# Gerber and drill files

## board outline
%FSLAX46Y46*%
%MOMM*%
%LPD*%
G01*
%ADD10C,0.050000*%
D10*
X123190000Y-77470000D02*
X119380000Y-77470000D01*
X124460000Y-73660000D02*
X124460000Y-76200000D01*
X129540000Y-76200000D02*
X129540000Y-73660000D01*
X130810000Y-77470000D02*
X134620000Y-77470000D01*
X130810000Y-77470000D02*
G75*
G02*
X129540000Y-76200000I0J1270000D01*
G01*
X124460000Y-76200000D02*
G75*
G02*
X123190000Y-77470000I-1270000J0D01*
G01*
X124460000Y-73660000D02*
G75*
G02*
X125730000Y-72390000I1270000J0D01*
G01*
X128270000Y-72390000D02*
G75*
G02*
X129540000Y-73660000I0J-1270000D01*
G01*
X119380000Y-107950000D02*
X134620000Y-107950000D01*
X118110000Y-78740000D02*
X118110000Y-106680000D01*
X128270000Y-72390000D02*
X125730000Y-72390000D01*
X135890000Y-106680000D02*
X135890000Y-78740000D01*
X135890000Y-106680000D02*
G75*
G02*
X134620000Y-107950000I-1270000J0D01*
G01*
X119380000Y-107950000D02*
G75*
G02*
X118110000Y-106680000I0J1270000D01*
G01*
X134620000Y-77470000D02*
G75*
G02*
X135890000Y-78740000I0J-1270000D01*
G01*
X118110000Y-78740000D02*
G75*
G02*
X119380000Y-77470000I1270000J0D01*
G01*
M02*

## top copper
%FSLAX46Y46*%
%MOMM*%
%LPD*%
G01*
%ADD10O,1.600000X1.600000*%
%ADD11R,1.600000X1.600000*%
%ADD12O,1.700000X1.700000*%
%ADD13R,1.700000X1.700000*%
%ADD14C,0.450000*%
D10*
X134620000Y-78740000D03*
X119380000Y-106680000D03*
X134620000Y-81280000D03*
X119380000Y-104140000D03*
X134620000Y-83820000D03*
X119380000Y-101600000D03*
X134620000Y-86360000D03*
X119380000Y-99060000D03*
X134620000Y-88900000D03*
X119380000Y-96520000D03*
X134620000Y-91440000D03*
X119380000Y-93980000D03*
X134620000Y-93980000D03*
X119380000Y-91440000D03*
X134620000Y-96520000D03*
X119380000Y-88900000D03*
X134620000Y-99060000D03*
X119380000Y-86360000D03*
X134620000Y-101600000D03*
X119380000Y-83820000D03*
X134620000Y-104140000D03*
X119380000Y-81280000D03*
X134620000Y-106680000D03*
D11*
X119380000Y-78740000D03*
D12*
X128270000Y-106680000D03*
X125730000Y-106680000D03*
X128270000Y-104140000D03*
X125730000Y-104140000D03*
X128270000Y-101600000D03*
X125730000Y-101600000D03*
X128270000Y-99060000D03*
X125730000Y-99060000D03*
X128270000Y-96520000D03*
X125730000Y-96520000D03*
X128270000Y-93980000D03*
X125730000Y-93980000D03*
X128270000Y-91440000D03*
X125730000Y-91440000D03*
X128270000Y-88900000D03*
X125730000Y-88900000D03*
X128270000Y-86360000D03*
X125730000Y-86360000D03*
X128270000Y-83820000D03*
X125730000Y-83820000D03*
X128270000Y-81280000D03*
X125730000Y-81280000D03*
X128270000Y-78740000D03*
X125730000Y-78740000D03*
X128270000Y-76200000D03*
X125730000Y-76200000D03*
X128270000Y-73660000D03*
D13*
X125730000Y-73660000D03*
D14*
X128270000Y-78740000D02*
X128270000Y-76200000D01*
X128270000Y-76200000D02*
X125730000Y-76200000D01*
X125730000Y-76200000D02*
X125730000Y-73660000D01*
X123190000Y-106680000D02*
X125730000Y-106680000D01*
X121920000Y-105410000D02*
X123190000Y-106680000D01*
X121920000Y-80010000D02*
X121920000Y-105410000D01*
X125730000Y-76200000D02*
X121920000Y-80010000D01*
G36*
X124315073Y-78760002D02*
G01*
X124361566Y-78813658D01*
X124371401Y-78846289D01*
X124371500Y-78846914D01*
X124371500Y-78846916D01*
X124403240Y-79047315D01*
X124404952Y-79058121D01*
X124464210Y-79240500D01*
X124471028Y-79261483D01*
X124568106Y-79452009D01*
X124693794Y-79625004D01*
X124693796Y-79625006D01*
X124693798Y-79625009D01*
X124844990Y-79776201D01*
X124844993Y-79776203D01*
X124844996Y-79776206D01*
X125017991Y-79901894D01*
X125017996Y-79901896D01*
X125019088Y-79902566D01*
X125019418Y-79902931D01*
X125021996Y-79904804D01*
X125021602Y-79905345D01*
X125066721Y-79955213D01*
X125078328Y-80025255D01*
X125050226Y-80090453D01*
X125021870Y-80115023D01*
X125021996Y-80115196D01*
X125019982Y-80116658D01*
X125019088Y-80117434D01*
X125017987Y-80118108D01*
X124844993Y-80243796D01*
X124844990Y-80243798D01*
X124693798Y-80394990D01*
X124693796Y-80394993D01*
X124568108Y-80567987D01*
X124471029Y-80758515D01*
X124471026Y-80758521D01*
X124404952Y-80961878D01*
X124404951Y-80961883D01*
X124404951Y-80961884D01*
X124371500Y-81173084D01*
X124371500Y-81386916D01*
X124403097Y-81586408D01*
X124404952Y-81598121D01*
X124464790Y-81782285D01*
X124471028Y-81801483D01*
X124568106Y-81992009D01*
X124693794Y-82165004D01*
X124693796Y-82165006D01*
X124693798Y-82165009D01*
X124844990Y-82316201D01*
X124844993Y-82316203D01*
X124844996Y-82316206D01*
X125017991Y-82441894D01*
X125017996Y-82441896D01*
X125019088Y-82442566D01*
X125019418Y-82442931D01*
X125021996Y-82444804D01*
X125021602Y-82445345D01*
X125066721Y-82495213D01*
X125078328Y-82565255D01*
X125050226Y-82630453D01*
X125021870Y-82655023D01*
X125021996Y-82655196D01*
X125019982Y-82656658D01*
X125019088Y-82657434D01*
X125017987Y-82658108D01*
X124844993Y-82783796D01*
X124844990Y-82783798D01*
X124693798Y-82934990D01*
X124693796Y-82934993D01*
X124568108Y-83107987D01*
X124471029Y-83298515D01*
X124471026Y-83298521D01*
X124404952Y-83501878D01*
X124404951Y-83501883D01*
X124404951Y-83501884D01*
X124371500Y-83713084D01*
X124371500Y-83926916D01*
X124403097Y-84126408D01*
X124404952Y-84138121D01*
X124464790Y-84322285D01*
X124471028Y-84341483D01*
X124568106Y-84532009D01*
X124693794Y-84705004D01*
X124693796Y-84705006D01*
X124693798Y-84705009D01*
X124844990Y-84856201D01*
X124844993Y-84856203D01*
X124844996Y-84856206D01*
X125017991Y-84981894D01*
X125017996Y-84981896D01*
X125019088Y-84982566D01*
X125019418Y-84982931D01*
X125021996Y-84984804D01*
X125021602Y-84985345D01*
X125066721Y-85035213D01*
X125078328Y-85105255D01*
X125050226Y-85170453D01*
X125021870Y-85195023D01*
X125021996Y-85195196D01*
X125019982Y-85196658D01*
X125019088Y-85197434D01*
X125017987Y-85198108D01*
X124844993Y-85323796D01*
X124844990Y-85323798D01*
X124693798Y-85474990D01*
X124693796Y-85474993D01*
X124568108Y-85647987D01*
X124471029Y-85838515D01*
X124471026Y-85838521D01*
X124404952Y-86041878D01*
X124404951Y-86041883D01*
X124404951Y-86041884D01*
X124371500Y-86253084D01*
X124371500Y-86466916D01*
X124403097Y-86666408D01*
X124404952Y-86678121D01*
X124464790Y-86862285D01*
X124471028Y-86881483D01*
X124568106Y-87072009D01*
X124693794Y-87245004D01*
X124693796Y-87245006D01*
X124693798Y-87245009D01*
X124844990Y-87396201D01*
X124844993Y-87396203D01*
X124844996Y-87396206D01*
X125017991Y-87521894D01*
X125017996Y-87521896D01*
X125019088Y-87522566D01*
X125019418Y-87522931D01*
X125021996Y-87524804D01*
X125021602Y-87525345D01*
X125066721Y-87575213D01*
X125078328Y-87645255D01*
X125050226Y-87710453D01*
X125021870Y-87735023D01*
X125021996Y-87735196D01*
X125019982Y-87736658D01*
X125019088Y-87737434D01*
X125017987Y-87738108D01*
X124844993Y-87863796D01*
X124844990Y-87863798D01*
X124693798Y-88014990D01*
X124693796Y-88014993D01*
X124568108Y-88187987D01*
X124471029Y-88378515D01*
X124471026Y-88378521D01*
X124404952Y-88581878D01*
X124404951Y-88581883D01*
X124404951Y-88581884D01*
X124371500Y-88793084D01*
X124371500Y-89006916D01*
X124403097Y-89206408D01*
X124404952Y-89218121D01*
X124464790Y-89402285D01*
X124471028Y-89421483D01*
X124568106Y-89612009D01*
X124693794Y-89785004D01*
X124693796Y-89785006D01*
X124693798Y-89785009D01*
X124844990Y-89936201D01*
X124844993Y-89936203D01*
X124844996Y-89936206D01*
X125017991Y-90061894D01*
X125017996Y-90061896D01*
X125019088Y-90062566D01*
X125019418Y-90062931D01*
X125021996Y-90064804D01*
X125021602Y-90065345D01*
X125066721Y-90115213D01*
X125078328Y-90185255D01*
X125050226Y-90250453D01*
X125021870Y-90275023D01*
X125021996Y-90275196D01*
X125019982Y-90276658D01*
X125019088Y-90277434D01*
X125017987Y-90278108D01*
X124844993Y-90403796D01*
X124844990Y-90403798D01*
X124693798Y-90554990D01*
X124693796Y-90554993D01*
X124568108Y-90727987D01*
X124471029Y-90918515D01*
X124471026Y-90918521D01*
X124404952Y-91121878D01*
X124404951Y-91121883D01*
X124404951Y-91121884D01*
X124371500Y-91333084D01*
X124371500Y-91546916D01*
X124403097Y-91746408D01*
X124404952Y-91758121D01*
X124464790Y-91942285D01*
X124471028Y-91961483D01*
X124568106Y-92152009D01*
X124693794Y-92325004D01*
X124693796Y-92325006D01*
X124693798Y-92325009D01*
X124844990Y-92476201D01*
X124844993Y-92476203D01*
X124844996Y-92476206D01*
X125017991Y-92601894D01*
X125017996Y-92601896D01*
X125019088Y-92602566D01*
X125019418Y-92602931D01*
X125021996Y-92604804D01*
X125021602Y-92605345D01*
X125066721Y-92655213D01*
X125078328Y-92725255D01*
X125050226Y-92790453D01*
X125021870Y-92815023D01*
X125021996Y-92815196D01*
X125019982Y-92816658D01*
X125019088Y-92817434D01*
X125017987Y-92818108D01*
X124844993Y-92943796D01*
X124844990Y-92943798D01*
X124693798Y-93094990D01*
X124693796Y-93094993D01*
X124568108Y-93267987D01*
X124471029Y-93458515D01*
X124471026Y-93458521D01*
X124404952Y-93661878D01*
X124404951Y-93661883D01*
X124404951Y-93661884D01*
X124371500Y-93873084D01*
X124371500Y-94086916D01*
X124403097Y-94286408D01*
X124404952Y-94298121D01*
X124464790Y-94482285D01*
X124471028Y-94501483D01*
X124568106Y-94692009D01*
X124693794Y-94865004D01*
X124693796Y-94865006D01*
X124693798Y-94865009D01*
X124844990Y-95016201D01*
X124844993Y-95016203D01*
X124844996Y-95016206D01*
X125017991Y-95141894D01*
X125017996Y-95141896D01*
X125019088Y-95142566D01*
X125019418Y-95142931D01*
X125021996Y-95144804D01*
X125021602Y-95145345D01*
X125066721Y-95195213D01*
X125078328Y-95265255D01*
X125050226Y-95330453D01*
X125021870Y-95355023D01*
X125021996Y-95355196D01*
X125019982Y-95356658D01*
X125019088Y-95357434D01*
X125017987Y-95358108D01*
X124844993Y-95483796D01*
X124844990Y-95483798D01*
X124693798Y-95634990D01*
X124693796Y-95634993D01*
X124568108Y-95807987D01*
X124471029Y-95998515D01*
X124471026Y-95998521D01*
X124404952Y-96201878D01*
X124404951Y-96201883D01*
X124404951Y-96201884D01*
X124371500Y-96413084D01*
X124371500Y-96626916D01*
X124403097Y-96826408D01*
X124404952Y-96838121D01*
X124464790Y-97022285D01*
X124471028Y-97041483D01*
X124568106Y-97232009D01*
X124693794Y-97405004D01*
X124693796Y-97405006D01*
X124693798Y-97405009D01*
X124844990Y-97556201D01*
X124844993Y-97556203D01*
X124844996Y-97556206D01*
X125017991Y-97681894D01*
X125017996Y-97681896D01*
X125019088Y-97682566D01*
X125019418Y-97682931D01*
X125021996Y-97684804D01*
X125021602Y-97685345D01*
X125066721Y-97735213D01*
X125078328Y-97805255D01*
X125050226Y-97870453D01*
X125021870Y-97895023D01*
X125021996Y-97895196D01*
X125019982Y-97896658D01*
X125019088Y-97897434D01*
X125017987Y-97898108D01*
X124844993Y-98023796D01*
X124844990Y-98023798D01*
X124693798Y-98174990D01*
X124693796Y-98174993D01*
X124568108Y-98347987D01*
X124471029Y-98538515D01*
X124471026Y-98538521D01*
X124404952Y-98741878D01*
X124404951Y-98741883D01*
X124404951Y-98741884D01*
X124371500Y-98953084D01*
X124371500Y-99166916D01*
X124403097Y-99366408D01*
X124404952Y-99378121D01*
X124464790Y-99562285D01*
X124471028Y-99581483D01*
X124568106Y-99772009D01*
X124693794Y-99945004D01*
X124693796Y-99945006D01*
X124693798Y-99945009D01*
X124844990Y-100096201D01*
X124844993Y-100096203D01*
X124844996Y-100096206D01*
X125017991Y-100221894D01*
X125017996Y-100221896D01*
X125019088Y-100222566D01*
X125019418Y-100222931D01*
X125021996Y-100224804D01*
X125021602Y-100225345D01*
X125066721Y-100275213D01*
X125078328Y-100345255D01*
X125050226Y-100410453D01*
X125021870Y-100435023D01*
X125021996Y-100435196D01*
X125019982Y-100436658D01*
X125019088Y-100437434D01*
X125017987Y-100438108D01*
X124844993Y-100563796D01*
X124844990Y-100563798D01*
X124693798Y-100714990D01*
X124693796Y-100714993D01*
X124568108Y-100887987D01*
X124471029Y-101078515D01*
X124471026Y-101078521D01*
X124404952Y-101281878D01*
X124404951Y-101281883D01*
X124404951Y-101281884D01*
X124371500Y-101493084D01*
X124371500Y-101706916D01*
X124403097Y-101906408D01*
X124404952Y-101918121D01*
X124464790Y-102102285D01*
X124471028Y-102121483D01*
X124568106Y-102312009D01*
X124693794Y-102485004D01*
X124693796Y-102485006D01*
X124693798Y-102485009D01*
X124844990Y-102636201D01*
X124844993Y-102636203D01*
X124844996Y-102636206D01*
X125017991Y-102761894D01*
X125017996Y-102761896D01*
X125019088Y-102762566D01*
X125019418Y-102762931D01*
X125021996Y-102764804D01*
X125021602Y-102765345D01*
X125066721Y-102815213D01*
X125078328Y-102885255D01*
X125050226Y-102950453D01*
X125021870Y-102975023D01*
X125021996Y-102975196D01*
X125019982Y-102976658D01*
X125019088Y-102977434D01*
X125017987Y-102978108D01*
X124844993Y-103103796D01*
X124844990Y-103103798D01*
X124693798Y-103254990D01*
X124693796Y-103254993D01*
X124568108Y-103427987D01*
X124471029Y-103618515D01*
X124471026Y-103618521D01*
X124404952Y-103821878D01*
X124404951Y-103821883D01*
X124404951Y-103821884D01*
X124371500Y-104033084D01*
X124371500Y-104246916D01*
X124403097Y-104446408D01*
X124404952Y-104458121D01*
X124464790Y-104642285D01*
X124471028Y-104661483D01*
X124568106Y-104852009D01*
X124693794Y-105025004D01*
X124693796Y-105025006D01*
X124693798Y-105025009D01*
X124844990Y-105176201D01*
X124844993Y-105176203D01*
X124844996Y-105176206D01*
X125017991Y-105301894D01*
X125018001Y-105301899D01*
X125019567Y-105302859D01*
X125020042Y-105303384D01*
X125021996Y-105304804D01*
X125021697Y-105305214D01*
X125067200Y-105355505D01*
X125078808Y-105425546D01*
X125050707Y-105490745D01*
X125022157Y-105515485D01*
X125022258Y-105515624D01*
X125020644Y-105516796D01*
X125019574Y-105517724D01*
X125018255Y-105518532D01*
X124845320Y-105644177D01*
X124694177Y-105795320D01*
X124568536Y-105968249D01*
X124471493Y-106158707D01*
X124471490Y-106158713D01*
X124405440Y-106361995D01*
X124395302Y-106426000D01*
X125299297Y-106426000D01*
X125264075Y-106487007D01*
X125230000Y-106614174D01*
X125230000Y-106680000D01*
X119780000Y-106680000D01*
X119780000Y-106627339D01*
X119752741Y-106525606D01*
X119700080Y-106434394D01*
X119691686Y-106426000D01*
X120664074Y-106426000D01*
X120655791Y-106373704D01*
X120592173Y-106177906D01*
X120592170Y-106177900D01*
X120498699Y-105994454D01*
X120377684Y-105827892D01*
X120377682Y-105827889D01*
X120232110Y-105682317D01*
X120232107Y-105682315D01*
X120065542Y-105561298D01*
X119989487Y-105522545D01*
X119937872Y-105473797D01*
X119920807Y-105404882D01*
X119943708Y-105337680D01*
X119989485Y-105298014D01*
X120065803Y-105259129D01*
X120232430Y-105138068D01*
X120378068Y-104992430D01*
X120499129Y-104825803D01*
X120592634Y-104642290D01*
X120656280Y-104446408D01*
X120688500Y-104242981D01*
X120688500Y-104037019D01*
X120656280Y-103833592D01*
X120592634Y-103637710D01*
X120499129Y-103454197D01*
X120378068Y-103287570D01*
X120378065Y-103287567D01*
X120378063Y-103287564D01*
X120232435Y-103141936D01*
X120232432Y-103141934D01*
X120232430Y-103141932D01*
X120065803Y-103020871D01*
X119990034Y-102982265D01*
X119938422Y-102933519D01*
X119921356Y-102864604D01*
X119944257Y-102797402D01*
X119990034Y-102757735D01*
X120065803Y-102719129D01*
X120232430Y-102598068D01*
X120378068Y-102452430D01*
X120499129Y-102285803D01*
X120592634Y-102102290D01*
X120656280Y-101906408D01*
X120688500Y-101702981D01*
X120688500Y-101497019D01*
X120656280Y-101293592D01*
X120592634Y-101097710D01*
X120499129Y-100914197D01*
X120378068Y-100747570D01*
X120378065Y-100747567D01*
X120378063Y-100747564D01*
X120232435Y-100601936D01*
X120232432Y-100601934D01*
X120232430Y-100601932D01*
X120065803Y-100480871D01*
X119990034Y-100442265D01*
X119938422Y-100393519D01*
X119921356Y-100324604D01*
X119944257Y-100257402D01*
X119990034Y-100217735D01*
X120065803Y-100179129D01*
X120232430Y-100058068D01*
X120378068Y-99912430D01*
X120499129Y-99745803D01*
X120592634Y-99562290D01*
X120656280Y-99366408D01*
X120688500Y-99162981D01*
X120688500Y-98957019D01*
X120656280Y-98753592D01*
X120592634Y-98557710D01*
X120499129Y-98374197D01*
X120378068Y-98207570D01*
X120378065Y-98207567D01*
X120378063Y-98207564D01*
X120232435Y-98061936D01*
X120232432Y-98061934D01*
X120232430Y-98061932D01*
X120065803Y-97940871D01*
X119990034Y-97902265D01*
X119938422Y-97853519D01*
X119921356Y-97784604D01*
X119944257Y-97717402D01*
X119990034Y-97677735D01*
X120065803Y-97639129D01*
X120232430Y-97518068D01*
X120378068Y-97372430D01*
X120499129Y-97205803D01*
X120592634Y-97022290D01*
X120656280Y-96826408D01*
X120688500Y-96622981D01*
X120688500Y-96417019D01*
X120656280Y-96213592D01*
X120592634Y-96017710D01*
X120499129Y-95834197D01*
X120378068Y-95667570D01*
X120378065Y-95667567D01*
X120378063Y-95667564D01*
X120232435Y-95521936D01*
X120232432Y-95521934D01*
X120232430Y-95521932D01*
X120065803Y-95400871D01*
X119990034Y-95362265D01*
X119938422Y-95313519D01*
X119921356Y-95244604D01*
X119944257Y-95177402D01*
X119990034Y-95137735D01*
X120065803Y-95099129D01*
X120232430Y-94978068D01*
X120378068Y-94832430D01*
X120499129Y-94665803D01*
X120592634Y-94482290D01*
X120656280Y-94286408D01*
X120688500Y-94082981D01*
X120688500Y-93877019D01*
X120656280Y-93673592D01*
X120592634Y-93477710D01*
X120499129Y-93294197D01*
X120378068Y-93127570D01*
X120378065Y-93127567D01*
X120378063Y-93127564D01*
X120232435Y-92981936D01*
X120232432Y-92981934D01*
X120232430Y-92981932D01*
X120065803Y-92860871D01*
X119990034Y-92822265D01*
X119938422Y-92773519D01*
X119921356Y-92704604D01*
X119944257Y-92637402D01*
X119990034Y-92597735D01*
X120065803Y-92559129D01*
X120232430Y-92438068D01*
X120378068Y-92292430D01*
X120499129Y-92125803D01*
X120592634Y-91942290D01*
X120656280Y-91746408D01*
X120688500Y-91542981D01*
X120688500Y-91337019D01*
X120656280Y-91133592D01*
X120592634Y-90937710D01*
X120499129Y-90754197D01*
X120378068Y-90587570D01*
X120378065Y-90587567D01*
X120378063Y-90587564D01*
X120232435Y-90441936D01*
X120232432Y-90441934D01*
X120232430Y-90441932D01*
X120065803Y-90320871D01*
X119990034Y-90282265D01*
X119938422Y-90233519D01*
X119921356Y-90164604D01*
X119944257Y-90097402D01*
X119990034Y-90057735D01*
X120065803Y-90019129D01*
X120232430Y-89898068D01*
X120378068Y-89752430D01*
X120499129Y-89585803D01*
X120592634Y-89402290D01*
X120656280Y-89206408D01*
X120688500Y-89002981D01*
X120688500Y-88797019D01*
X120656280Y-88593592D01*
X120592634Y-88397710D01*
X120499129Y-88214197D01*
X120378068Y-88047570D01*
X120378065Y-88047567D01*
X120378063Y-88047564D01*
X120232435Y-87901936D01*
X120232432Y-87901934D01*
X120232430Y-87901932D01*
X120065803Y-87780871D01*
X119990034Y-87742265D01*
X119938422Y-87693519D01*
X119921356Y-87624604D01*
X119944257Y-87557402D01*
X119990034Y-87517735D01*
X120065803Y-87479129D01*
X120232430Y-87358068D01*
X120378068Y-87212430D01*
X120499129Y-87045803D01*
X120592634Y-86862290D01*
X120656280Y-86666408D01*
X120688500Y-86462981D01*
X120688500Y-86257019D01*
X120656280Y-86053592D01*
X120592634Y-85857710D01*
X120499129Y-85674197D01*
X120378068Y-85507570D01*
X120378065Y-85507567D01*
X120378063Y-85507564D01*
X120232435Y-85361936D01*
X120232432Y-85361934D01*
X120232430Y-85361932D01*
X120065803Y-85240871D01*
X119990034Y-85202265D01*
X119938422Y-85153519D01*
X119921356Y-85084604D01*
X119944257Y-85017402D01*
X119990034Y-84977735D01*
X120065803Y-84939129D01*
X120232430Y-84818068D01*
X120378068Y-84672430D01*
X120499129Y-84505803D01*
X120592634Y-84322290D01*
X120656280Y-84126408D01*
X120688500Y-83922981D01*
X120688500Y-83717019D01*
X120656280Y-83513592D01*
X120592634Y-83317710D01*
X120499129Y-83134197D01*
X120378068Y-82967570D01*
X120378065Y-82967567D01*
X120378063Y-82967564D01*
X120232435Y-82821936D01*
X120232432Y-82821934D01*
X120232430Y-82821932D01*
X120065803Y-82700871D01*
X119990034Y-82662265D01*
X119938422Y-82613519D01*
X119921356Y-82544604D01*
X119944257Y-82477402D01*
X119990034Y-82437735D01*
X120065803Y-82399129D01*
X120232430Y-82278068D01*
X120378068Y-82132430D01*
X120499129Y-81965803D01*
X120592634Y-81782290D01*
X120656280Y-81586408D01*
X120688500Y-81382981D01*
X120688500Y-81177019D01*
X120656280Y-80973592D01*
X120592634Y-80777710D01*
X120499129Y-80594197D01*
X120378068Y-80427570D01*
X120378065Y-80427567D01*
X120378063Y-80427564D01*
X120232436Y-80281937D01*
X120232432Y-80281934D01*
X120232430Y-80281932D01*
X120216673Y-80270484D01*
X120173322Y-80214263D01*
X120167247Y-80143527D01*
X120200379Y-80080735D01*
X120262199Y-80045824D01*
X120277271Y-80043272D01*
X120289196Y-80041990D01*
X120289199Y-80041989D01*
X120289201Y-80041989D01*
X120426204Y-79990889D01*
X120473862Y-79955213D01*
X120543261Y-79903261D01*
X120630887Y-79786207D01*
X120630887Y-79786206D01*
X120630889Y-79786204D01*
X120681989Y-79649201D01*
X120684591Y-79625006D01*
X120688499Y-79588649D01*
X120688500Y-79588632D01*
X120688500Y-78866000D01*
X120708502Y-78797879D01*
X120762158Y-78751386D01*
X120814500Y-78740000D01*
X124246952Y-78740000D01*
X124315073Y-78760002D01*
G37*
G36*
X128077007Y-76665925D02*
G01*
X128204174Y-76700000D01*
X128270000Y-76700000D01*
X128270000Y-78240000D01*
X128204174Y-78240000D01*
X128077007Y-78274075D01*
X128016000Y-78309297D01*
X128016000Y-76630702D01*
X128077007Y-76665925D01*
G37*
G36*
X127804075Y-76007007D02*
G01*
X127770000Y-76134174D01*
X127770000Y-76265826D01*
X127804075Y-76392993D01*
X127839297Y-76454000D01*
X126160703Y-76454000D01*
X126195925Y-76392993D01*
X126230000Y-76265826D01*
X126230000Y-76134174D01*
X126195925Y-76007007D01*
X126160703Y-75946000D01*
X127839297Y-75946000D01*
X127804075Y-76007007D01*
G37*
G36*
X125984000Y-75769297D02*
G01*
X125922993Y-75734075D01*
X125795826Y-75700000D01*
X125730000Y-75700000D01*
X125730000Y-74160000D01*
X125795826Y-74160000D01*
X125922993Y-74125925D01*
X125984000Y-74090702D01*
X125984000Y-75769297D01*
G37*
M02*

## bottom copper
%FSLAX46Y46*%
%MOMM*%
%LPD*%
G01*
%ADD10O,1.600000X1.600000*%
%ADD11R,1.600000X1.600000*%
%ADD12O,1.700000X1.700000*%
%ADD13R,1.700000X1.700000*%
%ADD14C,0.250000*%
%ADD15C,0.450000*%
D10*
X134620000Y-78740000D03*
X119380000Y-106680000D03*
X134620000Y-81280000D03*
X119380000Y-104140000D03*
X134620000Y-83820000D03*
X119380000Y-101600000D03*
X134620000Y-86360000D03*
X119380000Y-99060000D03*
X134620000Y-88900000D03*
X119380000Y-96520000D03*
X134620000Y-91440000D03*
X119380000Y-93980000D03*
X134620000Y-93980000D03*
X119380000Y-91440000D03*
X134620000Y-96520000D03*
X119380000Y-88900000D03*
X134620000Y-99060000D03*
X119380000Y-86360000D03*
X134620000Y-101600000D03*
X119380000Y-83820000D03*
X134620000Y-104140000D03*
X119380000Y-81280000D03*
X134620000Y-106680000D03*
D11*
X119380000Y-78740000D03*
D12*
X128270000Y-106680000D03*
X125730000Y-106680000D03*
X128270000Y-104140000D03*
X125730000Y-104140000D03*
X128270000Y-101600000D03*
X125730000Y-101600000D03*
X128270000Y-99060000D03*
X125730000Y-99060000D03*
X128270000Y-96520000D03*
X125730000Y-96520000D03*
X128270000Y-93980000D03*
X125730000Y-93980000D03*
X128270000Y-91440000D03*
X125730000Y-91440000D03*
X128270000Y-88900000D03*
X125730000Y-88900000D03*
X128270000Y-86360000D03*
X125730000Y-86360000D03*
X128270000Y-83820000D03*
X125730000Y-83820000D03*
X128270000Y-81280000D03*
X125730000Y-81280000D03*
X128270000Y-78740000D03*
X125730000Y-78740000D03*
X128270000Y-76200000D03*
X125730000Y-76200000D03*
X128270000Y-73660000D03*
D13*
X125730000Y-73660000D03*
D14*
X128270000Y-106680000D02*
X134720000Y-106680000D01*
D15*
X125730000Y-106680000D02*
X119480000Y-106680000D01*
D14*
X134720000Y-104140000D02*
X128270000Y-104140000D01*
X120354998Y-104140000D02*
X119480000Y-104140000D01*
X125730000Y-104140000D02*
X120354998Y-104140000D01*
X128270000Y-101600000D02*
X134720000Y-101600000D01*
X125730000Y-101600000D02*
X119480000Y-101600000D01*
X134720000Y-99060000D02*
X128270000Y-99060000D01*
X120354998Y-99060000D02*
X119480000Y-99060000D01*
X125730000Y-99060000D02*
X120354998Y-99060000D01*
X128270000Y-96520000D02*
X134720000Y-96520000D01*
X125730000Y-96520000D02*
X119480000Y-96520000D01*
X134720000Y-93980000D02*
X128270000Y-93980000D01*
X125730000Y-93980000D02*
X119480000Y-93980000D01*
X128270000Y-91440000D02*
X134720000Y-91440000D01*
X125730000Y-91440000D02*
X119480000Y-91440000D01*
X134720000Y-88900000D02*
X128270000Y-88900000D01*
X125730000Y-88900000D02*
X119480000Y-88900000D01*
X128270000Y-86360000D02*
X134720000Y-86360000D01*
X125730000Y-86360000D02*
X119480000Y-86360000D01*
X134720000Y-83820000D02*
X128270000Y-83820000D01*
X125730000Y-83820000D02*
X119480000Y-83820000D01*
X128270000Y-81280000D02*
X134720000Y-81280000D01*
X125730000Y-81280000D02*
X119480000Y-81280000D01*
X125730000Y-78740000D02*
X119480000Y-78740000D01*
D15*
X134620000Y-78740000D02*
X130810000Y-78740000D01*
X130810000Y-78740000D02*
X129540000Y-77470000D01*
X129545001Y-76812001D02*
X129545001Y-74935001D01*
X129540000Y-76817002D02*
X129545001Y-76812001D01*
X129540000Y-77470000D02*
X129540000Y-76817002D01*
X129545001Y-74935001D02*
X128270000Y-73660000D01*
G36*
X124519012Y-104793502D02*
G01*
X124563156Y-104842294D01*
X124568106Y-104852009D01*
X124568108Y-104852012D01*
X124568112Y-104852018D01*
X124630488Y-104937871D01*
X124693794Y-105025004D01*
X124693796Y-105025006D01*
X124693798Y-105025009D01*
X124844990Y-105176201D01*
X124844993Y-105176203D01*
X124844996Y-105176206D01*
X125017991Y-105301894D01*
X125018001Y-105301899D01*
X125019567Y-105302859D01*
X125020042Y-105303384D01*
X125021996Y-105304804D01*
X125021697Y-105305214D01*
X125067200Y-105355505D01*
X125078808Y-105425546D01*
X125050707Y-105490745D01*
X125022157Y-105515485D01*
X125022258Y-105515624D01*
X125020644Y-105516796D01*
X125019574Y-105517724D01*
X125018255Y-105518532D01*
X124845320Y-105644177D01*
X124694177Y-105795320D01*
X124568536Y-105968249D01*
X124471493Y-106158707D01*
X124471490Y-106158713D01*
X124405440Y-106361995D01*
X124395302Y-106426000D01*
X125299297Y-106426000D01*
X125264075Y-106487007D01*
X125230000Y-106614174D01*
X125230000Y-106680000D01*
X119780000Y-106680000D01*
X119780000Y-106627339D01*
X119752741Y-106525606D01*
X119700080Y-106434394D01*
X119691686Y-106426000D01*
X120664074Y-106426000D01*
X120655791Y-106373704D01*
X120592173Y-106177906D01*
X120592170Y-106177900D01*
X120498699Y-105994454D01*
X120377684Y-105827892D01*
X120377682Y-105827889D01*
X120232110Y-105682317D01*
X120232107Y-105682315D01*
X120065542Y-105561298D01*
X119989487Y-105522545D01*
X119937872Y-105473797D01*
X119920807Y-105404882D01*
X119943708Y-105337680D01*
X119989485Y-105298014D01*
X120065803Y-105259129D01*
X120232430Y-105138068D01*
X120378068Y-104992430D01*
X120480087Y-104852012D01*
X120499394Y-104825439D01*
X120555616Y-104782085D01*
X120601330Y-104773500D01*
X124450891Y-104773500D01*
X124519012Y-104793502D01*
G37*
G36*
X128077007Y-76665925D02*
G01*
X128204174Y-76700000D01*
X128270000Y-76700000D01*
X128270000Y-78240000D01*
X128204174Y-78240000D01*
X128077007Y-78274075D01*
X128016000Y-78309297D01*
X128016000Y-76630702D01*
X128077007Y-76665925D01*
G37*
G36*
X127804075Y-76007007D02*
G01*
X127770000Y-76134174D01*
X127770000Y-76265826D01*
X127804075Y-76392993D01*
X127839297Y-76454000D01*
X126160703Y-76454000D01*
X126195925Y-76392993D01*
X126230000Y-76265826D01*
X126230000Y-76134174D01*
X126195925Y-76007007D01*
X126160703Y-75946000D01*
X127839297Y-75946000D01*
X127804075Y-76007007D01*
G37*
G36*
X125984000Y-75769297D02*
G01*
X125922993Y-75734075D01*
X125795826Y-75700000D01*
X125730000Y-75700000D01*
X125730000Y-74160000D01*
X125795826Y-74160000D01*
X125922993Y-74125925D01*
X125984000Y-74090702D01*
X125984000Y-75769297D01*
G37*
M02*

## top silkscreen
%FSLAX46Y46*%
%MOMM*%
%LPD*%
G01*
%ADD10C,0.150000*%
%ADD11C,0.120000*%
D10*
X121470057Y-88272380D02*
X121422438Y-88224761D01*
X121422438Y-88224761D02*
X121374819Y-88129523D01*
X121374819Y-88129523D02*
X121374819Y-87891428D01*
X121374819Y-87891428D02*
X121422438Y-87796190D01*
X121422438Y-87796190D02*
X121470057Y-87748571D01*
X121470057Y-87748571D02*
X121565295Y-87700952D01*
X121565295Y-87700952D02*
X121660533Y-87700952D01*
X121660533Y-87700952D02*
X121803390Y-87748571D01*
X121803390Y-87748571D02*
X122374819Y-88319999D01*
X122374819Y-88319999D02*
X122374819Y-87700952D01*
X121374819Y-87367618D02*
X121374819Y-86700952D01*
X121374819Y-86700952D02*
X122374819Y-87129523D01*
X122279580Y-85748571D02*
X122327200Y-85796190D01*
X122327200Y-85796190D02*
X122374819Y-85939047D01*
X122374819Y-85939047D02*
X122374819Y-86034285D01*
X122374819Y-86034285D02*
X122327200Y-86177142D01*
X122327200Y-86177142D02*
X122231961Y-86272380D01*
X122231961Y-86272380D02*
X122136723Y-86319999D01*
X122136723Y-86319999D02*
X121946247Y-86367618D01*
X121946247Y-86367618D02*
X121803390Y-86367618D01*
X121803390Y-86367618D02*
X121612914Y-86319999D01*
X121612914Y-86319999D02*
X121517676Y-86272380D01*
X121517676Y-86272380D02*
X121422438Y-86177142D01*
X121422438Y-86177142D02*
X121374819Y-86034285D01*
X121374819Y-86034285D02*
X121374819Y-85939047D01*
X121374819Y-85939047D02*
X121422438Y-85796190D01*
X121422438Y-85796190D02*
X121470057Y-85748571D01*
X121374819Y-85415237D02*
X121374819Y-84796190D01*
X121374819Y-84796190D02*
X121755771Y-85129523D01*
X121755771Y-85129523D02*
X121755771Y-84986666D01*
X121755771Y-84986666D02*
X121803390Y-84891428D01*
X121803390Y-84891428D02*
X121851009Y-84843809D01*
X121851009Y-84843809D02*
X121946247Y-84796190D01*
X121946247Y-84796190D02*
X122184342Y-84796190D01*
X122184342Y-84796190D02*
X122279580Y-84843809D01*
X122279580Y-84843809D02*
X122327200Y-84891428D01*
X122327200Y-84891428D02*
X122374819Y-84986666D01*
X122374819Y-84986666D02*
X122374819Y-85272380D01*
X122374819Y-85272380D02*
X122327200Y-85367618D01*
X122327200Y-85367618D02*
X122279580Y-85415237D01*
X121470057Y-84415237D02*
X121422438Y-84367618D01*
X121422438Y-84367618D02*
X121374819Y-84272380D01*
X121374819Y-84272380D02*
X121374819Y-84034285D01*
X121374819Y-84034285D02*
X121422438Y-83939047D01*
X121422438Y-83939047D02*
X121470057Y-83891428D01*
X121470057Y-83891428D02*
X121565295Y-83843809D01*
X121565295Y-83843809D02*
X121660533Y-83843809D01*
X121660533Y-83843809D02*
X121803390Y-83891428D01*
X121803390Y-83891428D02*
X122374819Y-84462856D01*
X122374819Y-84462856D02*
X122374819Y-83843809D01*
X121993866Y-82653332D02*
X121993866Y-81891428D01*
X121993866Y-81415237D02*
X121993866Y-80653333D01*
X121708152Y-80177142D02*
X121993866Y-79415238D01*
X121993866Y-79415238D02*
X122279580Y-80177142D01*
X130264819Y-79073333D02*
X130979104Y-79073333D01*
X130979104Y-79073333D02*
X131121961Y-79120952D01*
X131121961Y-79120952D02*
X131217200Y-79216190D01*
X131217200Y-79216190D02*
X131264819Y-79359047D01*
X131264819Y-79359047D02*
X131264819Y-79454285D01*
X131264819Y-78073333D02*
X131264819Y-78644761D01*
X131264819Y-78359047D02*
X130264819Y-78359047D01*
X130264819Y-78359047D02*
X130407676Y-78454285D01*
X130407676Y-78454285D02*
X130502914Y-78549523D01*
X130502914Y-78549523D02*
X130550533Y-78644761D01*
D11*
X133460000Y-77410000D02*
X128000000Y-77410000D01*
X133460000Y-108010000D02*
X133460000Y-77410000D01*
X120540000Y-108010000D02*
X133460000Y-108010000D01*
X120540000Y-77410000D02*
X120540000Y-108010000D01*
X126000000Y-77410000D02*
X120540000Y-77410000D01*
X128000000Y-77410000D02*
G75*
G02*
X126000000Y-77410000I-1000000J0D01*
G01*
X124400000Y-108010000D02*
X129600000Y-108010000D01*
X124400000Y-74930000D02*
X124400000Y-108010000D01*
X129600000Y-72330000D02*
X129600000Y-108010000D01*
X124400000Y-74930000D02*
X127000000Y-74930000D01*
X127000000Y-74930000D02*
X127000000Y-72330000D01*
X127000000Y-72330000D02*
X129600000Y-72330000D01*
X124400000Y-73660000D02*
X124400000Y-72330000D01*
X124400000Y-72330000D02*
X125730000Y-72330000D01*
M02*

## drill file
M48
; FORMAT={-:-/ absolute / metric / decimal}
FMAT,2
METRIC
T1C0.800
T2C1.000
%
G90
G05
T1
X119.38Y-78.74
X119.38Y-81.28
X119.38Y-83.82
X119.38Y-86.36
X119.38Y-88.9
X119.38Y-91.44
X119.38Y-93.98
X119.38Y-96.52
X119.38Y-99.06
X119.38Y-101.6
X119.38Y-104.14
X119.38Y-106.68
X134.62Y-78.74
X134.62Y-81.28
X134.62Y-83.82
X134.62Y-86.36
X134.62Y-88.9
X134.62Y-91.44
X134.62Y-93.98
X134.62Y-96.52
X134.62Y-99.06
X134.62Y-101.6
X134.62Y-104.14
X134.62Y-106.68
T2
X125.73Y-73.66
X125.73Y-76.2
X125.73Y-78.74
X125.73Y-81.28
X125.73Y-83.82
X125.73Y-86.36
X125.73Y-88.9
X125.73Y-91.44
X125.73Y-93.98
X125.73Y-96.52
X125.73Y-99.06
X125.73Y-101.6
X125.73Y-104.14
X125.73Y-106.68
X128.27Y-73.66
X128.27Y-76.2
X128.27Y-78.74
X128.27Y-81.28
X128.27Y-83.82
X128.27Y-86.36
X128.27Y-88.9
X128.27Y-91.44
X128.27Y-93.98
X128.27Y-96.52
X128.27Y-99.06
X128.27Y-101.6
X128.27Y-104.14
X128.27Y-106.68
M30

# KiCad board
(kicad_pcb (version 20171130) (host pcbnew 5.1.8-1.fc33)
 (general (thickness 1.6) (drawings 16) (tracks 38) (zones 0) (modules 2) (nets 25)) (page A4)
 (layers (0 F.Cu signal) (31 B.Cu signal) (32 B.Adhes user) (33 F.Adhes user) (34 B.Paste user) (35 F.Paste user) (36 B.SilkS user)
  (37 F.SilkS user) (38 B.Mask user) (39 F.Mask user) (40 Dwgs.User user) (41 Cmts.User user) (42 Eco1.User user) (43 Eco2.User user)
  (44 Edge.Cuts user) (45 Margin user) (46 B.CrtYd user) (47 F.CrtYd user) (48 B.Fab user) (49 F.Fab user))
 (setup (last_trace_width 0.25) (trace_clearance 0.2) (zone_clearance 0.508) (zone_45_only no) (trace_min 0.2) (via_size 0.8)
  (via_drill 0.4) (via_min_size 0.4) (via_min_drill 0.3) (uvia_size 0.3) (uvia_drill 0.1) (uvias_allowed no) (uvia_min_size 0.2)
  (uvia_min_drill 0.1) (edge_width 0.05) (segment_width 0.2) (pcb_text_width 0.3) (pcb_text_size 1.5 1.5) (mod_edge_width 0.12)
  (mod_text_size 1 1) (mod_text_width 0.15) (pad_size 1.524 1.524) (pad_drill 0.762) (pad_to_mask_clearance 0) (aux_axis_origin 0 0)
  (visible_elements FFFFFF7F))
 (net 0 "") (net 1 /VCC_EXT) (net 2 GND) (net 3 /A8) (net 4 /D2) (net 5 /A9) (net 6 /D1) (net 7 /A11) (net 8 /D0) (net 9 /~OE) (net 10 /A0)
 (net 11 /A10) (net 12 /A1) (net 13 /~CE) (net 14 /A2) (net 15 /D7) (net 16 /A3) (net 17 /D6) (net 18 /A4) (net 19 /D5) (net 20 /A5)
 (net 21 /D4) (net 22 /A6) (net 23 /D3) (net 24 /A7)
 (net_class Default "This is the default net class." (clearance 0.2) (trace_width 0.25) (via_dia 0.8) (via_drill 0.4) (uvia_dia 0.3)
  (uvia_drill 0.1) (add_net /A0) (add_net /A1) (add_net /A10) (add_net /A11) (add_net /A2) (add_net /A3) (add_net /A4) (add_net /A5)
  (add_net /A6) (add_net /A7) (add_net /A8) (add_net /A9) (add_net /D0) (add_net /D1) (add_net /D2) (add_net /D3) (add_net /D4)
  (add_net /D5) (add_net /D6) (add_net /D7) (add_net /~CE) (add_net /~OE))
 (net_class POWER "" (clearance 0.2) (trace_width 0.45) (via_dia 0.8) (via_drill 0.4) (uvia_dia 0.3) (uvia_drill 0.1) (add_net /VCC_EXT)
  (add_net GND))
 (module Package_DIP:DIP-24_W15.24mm (layer F.Cu) (at 119.38 78.74)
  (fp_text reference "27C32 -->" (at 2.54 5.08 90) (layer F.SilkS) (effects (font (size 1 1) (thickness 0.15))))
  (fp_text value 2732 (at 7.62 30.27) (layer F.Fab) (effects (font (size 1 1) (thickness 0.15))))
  (fp_line (start 14.08 -1.33) (end 8.62 -1.33) (layer F.SilkS) (width 0.12))
  (fp_line (start 14.08 29.27) (end 14.08 -1.33) (layer F.SilkS) (width 0.12))
  (fp_line (start 1.16 29.27) (end 14.08 29.27) (layer F.SilkS) (width 0.12))
  (fp_line (start 1.16 -1.33) (end 1.16 29.27) (layer F.SilkS) (width 0.12))
  (fp_line (start 6.62 -1.33) (end 1.16 -1.33) (layer F.SilkS) (width 0.12))
  (fp_arc (start 7.62 -1.33) (end 6.62 -1.33) (angle -180) (layer F.SilkS) (width 0.12))
  (pad 24 thru_hole oval (at 15.24 0) (size 1.6 1.6) (drill 0.8) (layers *.Cu *.Mask) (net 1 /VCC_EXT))
  (pad 12 thru_hole oval (at 0 27.94) (size 1.6 1.6) (drill 0.8) (layers *.Cu *.Mask) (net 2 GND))
  (pad 23 thru_hole oval (at 15.24 2.54) (size 1.6 1.6) (drill 0.8) (layers *.Cu *.Mask) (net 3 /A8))
  (pad 11 thru_hole oval (at 0 25.4) (size 1.6 1.6) (drill 0.8) (layers *.Cu *.Mask) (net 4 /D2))
  (pad 22 thru_hole oval (at 15.24 5.08) (size 1.6 1.6) (drill 0.8) (layers *.Cu *.Mask) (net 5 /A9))
  (pad 10 thru_hole oval (at 0 22.86) (size 1.6 1.6) (drill 0.8) (layers *.Cu *.Mask) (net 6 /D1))
  (pad 21 thru_hole oval (at 15.24 7.62) (size 1.6 1.6) (drill 0.8) (layers *.Cu *.Mask) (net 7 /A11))
  (pad 9 thru_hole oval (at 0 20.32) (size 1.6 1.6) (drill 0.8) (layers *.Cu *.Mask) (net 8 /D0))
  (pad 20 thru_hole oval (at 15.24 10.16) (size 1.6 1.6) (drill 0.8) (layers *.Cu *.Mask) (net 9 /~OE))
  (pad 8 thru_hole oval (at 0 17.78) (size 1.6 1.6) (drill 0.8) (layers *.Cu *.Mask) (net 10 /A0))
  (pad 19 thru_hole oval (at 15.24 12.7) (size 1.6 1.6) (drill 0.8) (layers *.Cu *.Mask) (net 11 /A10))
  (pad 7 thru_hole oval (at 0 15.24) (size 1.6 1.6) (drill 0.8) (layers *.Cu *.Mask) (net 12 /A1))
  (pad 18 thru_hole oval (at 15.24 15.24) (size 1.6 1.6) (drill 0.8) (layers *.Cu *.Mask) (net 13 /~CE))
  (pad 6 thru_hole oval (at 0 12.7) (size 1.6 1.6) (drill 0.8) (layers *.Cu *.Mask) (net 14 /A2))
  (pad 17 thru_hole oval (at 15.24 17.78) (size 1.6 1.6) (drill 0.8) (layers *.Cu *.Mask) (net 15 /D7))
  (pad 5 thru_hole oval (at 0 10.16) (size 1.6 1.6) (drill 0.8) (layers *.Cu *.Mask) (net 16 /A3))
  (pad 16 thru_hole oval (at 15.24 20.32) (size 1.6 1.6) (drill 0.8) (layers *.Cu *.Mask) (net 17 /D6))
  (pad 4 thru_hole oval (at 0 7.62) (size 1.6 1.6) (drill 0.8) (layers *.Cu *.Mask) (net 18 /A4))
  (pad 15 thru_hole oval (at 15.24 22.86) (size 1.6 1.6) (drill 0.8) (layers *.Cu *.Mask) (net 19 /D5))
  (pad 3 thru_hole oval (at 0 5.08) (size 1.6 1.6) (drill 0.8) (layers *.Cu *.Mask) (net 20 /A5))
  (pad 14 thru_hole oval (at 15.24 25.4) (size 1.6 1.6) (drill 0.8) (layers *.Cu *.Mask) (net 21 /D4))
  (pad 2 thru_hole oval (at 0 2.54) (size 1.6 1.6) (drill 0.8) (layers *.Cu *.Mask) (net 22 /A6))
  (pad 13 thru_hole oval (at 15.24 27.94) (size 1.6 1.6) (drill 0.8) (layers *.Cu *.Mask) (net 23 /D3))
  (pad 1 thru_hole rect (at 0 0) (size 1.6 1.6) (drill 0.8) (layers *.Cu *.Mask) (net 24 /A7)))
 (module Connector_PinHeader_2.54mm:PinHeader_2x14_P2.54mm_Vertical (layer F.Cu) (at 125.73 73.66)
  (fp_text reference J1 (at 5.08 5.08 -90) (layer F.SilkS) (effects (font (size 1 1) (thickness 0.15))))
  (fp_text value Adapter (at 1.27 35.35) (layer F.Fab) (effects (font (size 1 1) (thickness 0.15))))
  (fp_line (start -1.33 34.35) (end 3.87 34.35) (layer F.SilkS) (width 0.12))
  (fp_line (start -1.33 1.27) (end -1.33 34.35) (layer F.SilkS) (width 0.12))
  (fp_line (start 3.87 -1.33) (end 3.87 34.35) (layer F.SilkS) (width 0.12))
  (fp_line (start -1.33 1.27) (end 1.27 1.27) (layer F.SilkS) (width 0.12))
  (fp_line (start 1.27 1.27) (end 1.27 -1.33) (layer F.SilkS) (width 0.12))
  (fp_line (start 1.27 -1.33) (end 3.87 -1.33) (layer F.SilkS) (width 0.12))
  (fp_line (start -1.33 0) (end -1.33 -1.33) (layer F.SilkS) (width 0.12))
  (fp_line (start -1.33 -1.33) (end 0 -1.33) (layer F.SilkS) (width 0.12))
  (pad 28 thru_hole oval (at 2.54 33.02) (size 1.7 1.7) (drill 1) (layers *.Cu *.Mask) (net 23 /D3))
  (pad 27 thru_hole oval (at 0 33.02) (size 1.7 1.7) (drill 1) (layers *.Cu *.Mask) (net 2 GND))
  (pad 26 thru_hole oval (at 2.54 30.48) (size 1.7 1.7) (drill 1) (layers *.Cu *.Mask) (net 21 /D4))
  (pad 25 thru_hole oval (at 0 30.48) (size 1.7 1.7) (drill 1) (layers *.Cu *.Mask) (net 4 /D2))
  (pad 24 thru_hole oval (at 2.54 27.94) (size 1.7 1.7) (drill 1) (layers *.Cu *.Mask) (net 19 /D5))
  (pad 23 thru_hole oval (at 0 27.94) (size 1.7 1.7) (drill 1) (layers *.Cu *.Mask) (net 6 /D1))
  (pad 22 thru_hole oval (at 2.54 25.4) (size 1.7 1.7) (drill 1) (layers *.Cu *.Mask) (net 17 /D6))
  (pad 21 thru_hole oval (at 0 25.4) (size 1.7 1.7) (drill 1) (layers *.Cu *.Mask) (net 8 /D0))
  (pad 20 thru_hole oval (at 2.54 22.86) (size 1.7 1.7) (drill 1) (layers *.Cu *.Mask) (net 15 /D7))
  (pad 19 thru_hole oval (at 0 22.86) (size 1.7 1.7) (drill 1) (layers *.Cu *.Mask) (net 10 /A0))
  (pad 18 thru_hole oval (at 2.54 20.32) (size 1.7 1.7) (drill 1) (layers *.Cu *.Mask) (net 13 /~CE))
  (pad 17 thru_hole oval (at 0 20.32) (size 1.7 1.7) (drill 1) (layers *.Cu *.Mask) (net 12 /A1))
  (pad 16 thru_hole oval (at 2.54 17.78) (size 1.7 1.7) (drill 1) (layers *.Cu *.Mask) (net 11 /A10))
  (pad 15 thru_hole oval (at 0 17.78) (size 1.7 1.7) (drill 1) (layers *.Cu *.Mask) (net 14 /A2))
  (pad 14 thru_hole oval (at 2.54 15.24) (size 1.7 1.7) (drill 1) (layers *.Cu *.Mask) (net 9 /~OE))
  (pad 13 thru_hole oval (at 0 15.24) (size 1.7 1.7) (drill 1) (layers *.Cu *.Mask) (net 16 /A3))
  (pad 12 thru_hole oval (at 2.54 12.7) (size 1.7 1.7) (drill 1) (layers *.Cu *.Mask) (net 7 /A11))
  (pad 11 thru_hole oval (at 0 12.7) (size 1.7 1.7) (drill 1) (layers *.Cu *.Mask) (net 18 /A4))
  (pad 10 thru_hole oval (at 2.54 10.16) (size 1.7 1.7) (drill 1) (layers *.Cu *.Mask) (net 5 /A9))
  (pad 9 thru_hole oval (at 0 10.16) (size 1.7 1.7) (drill 1) (layers *.Cu *.Mask) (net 20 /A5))
  (pad 8 thru_hole oval (at 2.54 7.62) (size 1.7 1.7) (drill 1) (layers *.Cu *.Mask) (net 3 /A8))
  (pad 7 thru_hole oval (at 0 7.62) (size 1.7 1.7) (drill 1) (layers *.Cu *.Mask) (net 22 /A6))
  (pad 6 thru_hole oval (at 2.54 5.08) (size 1.7 1.7) (drill 1) (layers *.Cu *.Mask) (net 2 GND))
  (pad 5 thru_hole oval (at 0 5.08) (size 1.7 1.7) (drill 1) (layers *.Cu *.Mask) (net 24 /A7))
  (pad 4 thru_hole oval (at 2.54 2.54) (size 1.7 1.7) (drill 1) (layers *.Cu *.Mask) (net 2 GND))
  (pad 3 thru_hole oval (at 0 2.54) (size 1.7 1.7) (drill 1) (layers *.Cu *.Mask) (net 2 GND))
  (pad 2 thru_hole oval (at 2.54 0) (size 1.7 1.7) (drill 1) (layers *.Cu *.Mask) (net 1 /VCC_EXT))
  (pad 1 thru_hole rect (at 0 0) (size 1.7 1.7) (drill 1) (layers *.Cu *.Mask) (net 2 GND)))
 (gr_line (start 123.19 77.47) (end 119.38 77.47) (layer Edge.Cuts) (width 0.05))
 (gr_line (start 124.46 73.66) (end 124.46 76.2) (layer Edge.Cuts) (width 0.05))
 (gr_line (start 129.54 76.2) (end 129.54 73.66) (layer Edge.Cuts) (width 0.05))
 (gr_line (start 130.81 77.47) (end 134.62 77.47) (layer Edge.Cuts) (width 0.05))
 (gr_arc (start 130.81 76.2) (end 129.54 76.2) (angle -90) (layer Edge.Cuts) (width 0.05))
 (gr_arc (start 123.19 76.2) (end 123.19 77.47) (angle -90) (layer Edge.Cuts) (width 0.05))
 (gr_arc (start 125.73 73.66) (end 125.73 72.39) (angle -90) (layer Edge.Cuts) (width 0.05))
 (gr_arc (start 128.27 73.66) (end 129.54 73.66) (angle -90) (layer Edge.Cuts) (width 0.05))
 (gr_line (start 119.38 107.95) (end 134.62 107.95) (layer Edge.Cuts) (width 0.05))
 (gr_line (start 118.11 78.74) (end 118.11 106.68) (layer Edge.Cuts) (width 0.05))
 (gr_line (start 128.27 72.39) (end 125.73 72.39) (layer Edge.Cuts) (width 0.05))
 (gr_line (start 135.89 106.68) (end 135.89 78.74) (layer Edge.Cuts) (width 0.05))
 (gr_arc (start 134.62 106.68) (end 134.62 107.95) (angle -90) (layer Edge.Cuts) (width 0.05))
 (gr_arc (start 119.38 106.68) (end 118.11 106.68) (angle -90) (layer Edge.Cuts) (width 0.05))
 (gr_arc (start 134.62 78.74) (end 135.89 78.74) (angle -90) (layer Edge.Cuts) (width 0.05))
 (gr_arc (start 119.38 78.74) (end 119.38 77.47) (angle -90) (layer Edge.Cuts) (width 0.05))
 (segment (start 128.27 106.68) (end 134.72 106.68) (width 0.25) (layer B.Cu) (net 23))
 (segment (start 125.73 106.68) (end 119.48 106.68) (width 0.45) (layer B.Cu) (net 2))
 (segment (start 128.27 78.74) (end 128.27 76.2) (width 0.45) (layer F.Cu) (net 2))
 (segment (start 128.27 76.2) (end 125.73 76.2) (width 0.45) (layer F.Cu) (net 2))
 (segment (start 125.73 76.2) (end 125.73 73.66) (width 0.45) (layer F.Cu) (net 2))
 (segment (start 123.19 106.68) (end 125.73 106.68) (width 0.45) (layer F.Cu) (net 2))
 (segment (start 121.92 105.41) (end 123.19 106.68) (width 0.45) (layer F.Cu) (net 2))
 (segment (start 121.92 80.01) (end 121.92 105.41) (width 0.45) (layer F.Cu) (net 2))
 (segment (start 125.73 76.2) (end 121.92 80.01) (width 0.45) (layer F.Cu) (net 2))
 (segment (start 134.72 104.14) (end 128.27 104.14) (width 0.25) (layer B.Cu) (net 21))
 (segment (start 120.354998 104.14) (end 119.48 104.14) (width 0.25) (layer B.Cu) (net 4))
 (segment (start 125.73 104.14) (end 120.354998 104.14) (width 0.25) (layer B.Cu) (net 4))
 (segment (start 128.27 101.6) (end 134.72 101.6) (width 0.25) (layer B.Cu) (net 19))
 (segment (start 125.73 101.6) (end 119.48 101.6) (width 0.25) (layer B.Cu) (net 6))
 (segment (start 134.72 99.06) (end 128.27 99.06) (width 0.25) (layer B.Cu) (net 17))
 (segment (start 120.354998 99.06) (end 119.48 99.06) (width 0.25) (layer B.Cu) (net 8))
 (segment (start 125.73 99.06) (end 120.354998 99.06) (width 0.25) (layer B.Cu) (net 8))
 (segment (start 128.27 96.52) (end 134.72 96.52) (width 0.25) (layer B.Cu) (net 15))
 (segment (start 125.73 96.52) (end 119.48 96.52) (width 0.25) (layer B.Cu) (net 10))
 (segment (start 134.72 93.98) (end 128.27 93.98) (width 0.25) (layer B.Cu) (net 13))
 (segment (start 125.73 93.98) (end 119.48 93.98) (width 0.25) (layer B.Cu) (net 12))
 (segment (start 128.27 91.44) (end 134.72 91.44) (width 0.25) (layer B.Cu) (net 11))
 (segment (start 125.73 91.44) (end 119.48 91.44) (width 0.25) (layer B.Cu) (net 14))
 (segment (start 134.72 88.9) (end 128.27 88.9) (width 0.25) (layer B.Cu) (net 9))
 (segment (start 125.73 88.9) (end 119.48 88.9) (width 0.25) (layer B.Cu) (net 16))
 (segment (start 128.27 86.36) (end 134.72 86.36) (width 0.25) (layer B.Cu) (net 7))
 (segment (start 125.73 86.36) (end 119.48 86.36) (width 0.25) (layer B.Cu) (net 18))
 (segment (start 134.72 83.82) (end 128.27 83.82) (width 0.25) (layer B.Cu) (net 5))
 (segment (start 125.73 83.82) (end 119.48 83.82) (width 0.25) (layer B.Cu) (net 20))
 (segment (start 128.27 81.28) (end 134.72 81.28) (width 0.25) (layer B.Cu) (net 3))
 (segment (start 125.73 81.28) (end 119.48 81.28) (width 0.25) (layer B.Cu) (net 22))
 (segment (start 125.73 78.74) (end 119.48 78.74) (width 0.25) (layer B.Cu) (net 24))
 (segment (start 134.62 78.74) (end 130.81 78.74) (width 0.45) (layer B.Cu) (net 1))
 (segment (start 130.81 78.74) (end 129.54 77.47) (width 0.45) (layer B.Cu) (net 1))
 (segment (start 129.545001 76.812001) (end 129.545001 74.935001) (width 0.45) (layer B.Cu) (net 1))
 (segment (start 129.54 76.817002) (end 129.545001 76.812001) (width 0.45) (layer B.Cu) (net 1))
 (segment (start 129.54 77.47) (end 129.54 76.817002) (width 0.45) (layer B.Cu) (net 1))
 (segment (start 129.545001 74.935001) (end 128.27 73.66) (width 0.45) (layer B.Cu) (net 1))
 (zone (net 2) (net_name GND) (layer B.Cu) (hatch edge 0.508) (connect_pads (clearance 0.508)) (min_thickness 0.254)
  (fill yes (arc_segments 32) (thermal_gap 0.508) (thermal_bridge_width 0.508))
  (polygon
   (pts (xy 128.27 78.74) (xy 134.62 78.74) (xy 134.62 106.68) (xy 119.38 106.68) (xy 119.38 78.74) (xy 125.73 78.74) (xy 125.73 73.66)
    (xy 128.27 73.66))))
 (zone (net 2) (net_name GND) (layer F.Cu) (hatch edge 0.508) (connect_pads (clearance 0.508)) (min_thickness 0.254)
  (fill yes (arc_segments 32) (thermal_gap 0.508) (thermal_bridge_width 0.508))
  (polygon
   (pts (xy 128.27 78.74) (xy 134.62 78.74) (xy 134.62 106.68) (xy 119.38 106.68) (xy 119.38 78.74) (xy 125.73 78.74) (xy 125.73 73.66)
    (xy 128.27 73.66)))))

